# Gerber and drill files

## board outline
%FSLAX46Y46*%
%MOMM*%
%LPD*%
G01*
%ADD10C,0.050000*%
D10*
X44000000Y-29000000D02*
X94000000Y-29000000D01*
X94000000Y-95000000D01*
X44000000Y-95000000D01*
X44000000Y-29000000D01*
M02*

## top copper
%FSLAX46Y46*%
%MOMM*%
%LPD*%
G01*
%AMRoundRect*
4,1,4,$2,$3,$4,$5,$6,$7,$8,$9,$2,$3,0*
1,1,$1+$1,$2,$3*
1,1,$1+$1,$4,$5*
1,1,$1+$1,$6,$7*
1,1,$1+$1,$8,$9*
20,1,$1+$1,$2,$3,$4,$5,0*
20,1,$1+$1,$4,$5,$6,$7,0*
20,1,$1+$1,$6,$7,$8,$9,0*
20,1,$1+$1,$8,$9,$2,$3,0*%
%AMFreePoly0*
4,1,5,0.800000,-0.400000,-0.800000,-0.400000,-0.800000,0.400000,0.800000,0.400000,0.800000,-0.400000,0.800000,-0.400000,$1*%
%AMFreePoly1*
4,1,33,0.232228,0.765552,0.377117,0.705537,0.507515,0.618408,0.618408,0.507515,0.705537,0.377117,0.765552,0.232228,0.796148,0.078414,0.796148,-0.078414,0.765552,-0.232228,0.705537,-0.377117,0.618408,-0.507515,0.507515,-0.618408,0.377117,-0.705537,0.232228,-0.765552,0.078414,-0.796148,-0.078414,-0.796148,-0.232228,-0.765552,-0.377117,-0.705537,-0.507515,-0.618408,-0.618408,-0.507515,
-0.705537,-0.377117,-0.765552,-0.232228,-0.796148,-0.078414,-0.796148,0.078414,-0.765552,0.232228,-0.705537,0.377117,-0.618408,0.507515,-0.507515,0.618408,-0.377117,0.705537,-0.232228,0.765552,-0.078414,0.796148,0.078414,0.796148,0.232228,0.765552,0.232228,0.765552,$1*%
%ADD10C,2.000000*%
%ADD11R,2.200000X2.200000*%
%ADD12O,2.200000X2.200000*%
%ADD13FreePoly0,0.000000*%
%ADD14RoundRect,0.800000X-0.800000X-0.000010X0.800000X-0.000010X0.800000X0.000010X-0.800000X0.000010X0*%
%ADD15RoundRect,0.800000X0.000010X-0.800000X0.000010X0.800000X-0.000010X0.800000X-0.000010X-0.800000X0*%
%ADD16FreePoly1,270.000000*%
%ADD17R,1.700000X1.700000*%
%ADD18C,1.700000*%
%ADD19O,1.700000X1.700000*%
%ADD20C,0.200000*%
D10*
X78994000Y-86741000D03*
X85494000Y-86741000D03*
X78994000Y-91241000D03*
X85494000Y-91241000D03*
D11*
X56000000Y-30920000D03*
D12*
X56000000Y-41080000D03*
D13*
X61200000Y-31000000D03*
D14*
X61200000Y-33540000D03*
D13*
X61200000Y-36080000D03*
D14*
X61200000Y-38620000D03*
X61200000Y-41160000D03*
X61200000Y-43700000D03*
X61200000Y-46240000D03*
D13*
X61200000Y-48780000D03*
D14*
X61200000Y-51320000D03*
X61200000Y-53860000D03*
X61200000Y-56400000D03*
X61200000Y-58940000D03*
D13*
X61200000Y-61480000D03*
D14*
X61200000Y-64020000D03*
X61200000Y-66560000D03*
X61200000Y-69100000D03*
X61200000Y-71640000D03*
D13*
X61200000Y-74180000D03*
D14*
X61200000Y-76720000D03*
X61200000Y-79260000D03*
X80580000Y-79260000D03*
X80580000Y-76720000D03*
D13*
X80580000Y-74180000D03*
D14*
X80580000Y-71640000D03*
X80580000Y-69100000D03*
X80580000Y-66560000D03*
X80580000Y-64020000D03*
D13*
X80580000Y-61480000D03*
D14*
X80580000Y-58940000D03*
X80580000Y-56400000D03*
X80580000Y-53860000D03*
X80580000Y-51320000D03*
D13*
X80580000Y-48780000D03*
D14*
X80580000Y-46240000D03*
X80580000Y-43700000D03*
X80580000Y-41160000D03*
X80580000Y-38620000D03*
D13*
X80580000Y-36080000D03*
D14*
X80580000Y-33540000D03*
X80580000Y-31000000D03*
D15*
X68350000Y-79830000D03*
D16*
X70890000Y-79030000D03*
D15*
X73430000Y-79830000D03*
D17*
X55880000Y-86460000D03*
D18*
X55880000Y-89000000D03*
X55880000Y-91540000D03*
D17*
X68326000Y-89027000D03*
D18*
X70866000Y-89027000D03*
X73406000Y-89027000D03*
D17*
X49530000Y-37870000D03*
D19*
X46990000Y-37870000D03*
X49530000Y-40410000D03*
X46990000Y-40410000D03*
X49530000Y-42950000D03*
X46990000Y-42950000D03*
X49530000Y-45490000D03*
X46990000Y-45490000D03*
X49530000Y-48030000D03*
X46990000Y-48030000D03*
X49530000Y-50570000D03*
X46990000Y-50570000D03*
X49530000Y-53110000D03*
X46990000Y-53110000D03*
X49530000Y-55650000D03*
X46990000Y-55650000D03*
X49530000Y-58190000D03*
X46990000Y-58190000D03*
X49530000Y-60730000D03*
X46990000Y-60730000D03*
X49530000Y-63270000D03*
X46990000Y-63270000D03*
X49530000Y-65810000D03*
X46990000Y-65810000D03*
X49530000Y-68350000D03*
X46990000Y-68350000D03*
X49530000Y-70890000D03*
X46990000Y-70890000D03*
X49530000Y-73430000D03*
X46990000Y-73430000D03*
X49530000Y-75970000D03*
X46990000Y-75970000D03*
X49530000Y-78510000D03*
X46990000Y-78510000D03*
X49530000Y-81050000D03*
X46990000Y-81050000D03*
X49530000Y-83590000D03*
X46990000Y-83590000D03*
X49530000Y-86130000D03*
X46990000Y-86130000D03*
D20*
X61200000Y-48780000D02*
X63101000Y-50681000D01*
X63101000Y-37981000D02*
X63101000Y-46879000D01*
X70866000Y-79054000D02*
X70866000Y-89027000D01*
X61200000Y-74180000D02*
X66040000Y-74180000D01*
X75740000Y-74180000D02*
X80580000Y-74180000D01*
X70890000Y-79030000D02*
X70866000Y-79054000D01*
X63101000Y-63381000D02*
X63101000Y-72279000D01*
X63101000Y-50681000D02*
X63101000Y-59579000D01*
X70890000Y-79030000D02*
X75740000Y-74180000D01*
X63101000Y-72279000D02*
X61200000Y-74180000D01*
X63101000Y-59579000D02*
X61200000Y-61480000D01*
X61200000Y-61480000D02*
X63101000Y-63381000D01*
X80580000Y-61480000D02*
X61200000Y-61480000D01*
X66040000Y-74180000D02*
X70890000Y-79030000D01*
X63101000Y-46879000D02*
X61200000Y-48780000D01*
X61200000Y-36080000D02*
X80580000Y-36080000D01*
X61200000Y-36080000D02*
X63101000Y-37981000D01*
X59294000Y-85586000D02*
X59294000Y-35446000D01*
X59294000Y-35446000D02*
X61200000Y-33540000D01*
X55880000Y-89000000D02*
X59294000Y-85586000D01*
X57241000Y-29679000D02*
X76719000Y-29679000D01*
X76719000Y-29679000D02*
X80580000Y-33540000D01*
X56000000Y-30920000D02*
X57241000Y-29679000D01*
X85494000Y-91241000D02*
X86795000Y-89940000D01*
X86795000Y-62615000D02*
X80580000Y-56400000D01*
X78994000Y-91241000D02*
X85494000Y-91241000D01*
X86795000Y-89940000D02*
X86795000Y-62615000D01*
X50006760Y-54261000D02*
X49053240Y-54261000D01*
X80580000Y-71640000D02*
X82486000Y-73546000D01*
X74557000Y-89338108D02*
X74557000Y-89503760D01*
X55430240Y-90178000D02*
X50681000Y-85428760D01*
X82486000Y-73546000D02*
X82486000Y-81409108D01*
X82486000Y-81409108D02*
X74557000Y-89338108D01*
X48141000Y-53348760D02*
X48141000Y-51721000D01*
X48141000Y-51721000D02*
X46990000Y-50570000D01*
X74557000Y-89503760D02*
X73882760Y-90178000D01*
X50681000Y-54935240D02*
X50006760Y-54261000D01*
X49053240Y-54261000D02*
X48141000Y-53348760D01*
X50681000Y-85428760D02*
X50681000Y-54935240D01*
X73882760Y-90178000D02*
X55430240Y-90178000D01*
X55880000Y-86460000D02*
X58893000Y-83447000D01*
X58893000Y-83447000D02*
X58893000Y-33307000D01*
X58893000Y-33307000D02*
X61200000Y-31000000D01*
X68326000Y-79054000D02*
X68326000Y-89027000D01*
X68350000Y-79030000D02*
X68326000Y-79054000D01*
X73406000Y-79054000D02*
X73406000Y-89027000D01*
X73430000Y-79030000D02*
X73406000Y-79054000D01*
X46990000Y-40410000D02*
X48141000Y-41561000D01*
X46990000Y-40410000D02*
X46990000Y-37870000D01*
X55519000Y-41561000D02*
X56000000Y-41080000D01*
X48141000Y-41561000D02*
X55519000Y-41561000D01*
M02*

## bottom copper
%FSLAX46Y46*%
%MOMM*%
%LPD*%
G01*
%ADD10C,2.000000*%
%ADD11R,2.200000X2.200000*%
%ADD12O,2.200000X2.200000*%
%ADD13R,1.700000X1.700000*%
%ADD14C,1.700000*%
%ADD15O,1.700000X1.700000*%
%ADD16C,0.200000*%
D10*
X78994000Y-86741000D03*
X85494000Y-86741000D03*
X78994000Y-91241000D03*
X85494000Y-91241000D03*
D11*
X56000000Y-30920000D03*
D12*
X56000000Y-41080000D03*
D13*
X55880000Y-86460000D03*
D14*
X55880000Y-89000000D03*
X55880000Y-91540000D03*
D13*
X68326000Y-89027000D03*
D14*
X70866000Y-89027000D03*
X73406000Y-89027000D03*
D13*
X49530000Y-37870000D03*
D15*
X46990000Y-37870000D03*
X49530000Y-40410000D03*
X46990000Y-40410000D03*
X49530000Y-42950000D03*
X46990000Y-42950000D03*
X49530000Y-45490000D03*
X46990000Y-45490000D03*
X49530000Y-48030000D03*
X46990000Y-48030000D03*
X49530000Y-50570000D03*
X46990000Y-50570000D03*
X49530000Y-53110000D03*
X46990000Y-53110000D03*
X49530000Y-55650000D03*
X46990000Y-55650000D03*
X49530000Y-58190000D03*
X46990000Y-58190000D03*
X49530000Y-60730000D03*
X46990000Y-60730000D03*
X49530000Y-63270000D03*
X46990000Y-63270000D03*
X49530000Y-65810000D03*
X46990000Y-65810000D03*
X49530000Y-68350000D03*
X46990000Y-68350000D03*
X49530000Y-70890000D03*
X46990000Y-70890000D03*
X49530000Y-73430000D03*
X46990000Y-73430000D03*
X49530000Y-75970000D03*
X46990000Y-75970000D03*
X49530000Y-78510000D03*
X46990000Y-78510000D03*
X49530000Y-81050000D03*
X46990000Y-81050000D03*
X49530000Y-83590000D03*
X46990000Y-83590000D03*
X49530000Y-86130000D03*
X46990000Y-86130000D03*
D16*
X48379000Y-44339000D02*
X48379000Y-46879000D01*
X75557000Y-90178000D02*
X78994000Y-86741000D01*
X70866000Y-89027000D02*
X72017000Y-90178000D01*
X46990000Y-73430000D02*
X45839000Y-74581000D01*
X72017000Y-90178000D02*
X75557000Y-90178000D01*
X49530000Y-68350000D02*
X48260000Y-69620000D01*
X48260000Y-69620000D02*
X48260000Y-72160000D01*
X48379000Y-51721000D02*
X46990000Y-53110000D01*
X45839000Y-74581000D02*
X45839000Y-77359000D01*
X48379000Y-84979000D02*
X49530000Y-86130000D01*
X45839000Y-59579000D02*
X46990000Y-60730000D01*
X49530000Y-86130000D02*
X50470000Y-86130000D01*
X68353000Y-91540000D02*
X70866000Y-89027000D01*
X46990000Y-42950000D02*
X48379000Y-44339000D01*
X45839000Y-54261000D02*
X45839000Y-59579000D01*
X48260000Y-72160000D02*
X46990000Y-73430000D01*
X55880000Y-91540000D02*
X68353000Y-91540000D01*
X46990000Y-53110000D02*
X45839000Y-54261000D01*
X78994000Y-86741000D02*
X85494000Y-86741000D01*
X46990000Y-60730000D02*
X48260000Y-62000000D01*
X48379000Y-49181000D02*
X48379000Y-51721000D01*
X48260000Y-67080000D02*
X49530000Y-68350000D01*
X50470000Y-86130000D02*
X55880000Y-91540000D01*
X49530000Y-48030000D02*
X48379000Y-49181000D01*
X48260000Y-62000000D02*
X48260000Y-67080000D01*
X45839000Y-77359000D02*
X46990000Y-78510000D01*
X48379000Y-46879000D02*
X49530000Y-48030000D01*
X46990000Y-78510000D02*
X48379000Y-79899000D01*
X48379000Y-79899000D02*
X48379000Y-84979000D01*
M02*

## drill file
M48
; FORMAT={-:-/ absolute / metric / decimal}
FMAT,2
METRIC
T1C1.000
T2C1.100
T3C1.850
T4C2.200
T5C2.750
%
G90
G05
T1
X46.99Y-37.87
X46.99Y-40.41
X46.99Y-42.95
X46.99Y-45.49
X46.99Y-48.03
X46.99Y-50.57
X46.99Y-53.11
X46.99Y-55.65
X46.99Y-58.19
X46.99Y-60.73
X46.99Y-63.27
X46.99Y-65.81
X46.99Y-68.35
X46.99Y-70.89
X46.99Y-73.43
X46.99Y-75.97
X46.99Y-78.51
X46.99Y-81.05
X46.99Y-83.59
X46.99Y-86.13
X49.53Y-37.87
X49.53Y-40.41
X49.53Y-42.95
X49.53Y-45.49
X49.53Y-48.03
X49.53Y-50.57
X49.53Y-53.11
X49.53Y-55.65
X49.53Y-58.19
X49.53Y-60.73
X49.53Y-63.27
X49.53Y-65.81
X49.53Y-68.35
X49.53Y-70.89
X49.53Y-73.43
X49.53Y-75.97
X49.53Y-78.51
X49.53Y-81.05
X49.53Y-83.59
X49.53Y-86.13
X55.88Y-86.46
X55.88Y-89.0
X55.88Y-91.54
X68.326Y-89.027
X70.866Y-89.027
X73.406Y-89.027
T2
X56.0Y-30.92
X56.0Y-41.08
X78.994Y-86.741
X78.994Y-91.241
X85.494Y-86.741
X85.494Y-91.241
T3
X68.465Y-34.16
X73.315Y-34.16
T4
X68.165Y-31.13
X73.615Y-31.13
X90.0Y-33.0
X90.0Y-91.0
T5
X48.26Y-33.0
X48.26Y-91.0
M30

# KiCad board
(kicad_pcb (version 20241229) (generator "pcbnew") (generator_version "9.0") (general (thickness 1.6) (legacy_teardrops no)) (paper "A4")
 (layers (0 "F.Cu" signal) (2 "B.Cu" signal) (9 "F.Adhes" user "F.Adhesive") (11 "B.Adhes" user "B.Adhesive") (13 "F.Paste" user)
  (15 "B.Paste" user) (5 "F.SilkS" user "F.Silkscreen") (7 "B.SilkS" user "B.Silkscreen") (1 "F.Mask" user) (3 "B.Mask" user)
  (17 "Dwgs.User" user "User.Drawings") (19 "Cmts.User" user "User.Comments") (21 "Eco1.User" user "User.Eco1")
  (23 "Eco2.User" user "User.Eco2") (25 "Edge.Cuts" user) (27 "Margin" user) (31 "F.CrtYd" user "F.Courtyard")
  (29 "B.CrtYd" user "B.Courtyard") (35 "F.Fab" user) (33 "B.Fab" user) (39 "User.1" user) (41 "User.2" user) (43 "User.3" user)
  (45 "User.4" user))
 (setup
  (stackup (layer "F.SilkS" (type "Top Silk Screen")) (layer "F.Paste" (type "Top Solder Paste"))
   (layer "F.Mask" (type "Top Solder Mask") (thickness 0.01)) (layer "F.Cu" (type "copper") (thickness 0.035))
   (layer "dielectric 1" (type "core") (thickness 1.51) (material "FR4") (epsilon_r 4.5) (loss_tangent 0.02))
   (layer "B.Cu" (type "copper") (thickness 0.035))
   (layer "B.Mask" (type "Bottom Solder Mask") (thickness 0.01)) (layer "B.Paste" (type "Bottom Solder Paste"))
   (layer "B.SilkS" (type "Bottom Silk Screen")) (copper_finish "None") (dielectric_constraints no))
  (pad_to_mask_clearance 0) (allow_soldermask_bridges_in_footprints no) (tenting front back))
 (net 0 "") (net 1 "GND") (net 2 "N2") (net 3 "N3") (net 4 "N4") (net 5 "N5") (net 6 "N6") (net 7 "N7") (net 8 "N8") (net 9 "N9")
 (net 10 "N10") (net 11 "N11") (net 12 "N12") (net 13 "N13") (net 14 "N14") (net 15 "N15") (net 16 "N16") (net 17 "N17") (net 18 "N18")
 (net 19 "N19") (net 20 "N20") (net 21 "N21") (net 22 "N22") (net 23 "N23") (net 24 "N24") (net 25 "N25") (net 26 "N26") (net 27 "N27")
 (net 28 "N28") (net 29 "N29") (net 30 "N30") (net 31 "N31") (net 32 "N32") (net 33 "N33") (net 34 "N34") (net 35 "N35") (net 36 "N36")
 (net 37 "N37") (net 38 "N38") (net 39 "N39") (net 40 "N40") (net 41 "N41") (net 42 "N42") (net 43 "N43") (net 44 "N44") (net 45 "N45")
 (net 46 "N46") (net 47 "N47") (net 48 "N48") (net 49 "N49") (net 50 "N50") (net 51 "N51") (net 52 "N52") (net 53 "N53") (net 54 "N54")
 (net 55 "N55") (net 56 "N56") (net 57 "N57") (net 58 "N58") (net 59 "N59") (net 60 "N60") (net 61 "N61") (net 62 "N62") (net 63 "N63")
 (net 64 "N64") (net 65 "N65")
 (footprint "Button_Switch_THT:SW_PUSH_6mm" (layer "F.Cu") (at 78.994 86.741)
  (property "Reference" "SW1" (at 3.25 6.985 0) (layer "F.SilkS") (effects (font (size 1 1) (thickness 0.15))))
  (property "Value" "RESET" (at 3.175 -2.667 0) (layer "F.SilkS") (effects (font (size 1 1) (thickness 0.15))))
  (pad "1" thru_hole circle (at 0 0 90) (size 2 2) (drill 1.1) (layers "*.Cu" "*.Mask") (remove_unused_layers no) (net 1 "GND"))
  (pad "1" thru_hole circle (at 6.5 0 90) (size 2 2) (drill 1.1) (layers "*.Cu" "*.Mask") (remove_unused_layers no) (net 1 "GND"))
  (pad "2" thru_hole circle (at 0 4.5 90) (size 2 2) (drill 1.1) (layers "*.Cu" "*.Mask") (remove_unused_layers no) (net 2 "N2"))
  (pad "2" thru_hole circle (at 6.5 4.5 90) (size 2 2) (drill 1.1) (layers "*.Cu" "*.Mask") (remove_unused_layers no) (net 2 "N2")))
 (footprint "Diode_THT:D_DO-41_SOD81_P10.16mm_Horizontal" (layer "F.Cu") (at 56 30.92 -90)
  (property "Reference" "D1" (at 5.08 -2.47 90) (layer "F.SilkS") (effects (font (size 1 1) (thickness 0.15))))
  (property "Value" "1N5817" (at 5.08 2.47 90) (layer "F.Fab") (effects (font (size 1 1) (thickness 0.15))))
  (pad "1" thru_hole rect (at 0 0 270) (size 2.2 2.2) (drill 1.1) (layers "*.Cu" "*.Mask") (remove_unused_layers no) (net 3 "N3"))
  (pad "2" thru_hole oval (at 10.16 0 270) (size 2.2 2.2) (drill 1.1) (layers "*.Cu" "*.Mask") (remove_unused_layers no) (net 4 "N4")))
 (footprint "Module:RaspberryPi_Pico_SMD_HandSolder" (layer "F.Cu") (at 70.89 55.13)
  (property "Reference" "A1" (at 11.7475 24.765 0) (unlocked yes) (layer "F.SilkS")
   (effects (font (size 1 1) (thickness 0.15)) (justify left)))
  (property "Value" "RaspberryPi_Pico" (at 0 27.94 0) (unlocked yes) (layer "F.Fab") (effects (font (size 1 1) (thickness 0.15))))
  (pad "" smd rect (at -8.89 -24.13) (size 3.8 2.2) (drill (offset -0.8 0)) (layers "F.Paste"))
  (pad "" smd rect (at -8.89 -21.59) (size 3.8 2.2) (drill (offset -0.8 0)) (layers "F.Paste"))
  (pad "" smd rect (at -8.89 -19.05) (size 3.8 2.2) (drill (offset -0.8 0)) (layers "F.Paste"))
  (pad "" smd rect (at -8.89 -16.51) (size 3.8 2.2) (drill (offset -0.8 0)) (layers "F.Paste"))
  (pad "" smd rect (at -8.89 -13.97) (size 3.8 2.2) (drill (offset -0.8 0)) (layers "F.Paste"))
  (pad "" smd rect (at -8.89 -11.43) (size 3.8 2.2) (drill (offset -0.8 0)) (layers "F.Paste"))
  (pad "" smd rect (at -8.89 -8.89) (size 3.8 2.2) (drill (offset -0.8 0)) (layers "F.Paste"))
  (pad "" smd rect (at -8.89 -6.35) (size 3.8 2.2) (drill (offset -0.8 0)) (layers "F.Paste"))
  (pad "" smd rect (at -8.89 -3.81) (size 3.8 2.2) (drill (offset -0.8 0)) (layers "F.Paste"))
  (pad "" smd rect (at -8.89 -1.27) (size 3.8 2.2) (drill (offset -0.8 0)) (layers "F.Paste"))
  (pad "" smd rect (at -8.89 1.27) (size 3.8 2.2) (drill (offset -0.8 0)) (layers "F.Paste"))
  (pad "" smd rect (at -8.89 3.81) (size 3.8 2.2) (drill (offset -0.8 0)) (layers "F.Paste"))
  (pad "" smd rect (at -8.89 6.35) (size 3.8 2.2) (drill (offset -0.8 0)) (layers "F.Paste"))
  (pad "" smd rect (at -8.89 8.89) (size 3.8 2.2) (drill (offset -0.8 0)) (layers "F.Paste"))
  (pad "" smd rect (at -8.89 11.43) (size 3.8 2.2) (drill (offset -0.8 0)) (layers "F.Paste"))
  (pad "" smd rect (at -8.89 13.97) (size 3.8 2.2) (drill (offset -0.8 0)) (layers "F.Paste"))
  (pad "" smd rect (at -8.89 16.51) (size 3.8 2.2) (drill (offset -0.8 0)) (layers "F.Paste"))
  (pad "" smd rect (at -8.89 19.05) (size 3.8 2.2) (drill (offset -0.8 0)) (layers "F.Paste"))
  (pad "" smd rect (at -8.89 21.59) (size 3.8 2.2) (drill (offset -0.8 0)) (layers "F.Paste"))
  (pad "" smd rect (at -8.89 24.13) (size 3.8 2.2) (drill (offset -0.8 0)) (layers "F.Paste"))
  (pad "" np_thru_hole circle (at -2.725 -24) (size 2.2 2.2) (drill 2.2) (layers "*.Mask"))
  (pad "" smd rect (at -2.54 23.9) (size 2.2 3.8) (drill (offset 0 0.8)) (layers "F.Paste"))
  (pad "" np_thru_hole circle (at -2.425 -20.97) (size 1.85 1.85) (drill 1.85) (layers "*.Mask"))
  (pad "" smd rect (at 0 23.9) (size 2.2 3.8) (drill (offset 0 0.8)) (layers "F.Paste"))
  (pad "" np_thru_hole circle (at 2.425 -20.97) (size 1.85 1.85) (drill 1.85) (layers "*.Mask"))
  (pad "" smd rect (at 2.54 23.9) (size 2.2 3.8) (drill (offset 0 0.8)) (layers "F.Paste"))
  (pad "" np_thru_hole circle (at 2.725 -24) (size 2.2 2.2) (drill 2.2) (layers "*.Mask"))
  (pad "" smd rect (at 8.89 -24.13) (size 3.8 2.2) (drill (offset 0.8 0)) (layers "F.Paste"))
  (pad "" smd rect (at 8.89 -21.59) (size 3.8 2.2) (drill (offset 0.8 0)) (layers "F.Paste"))
  (pad "" smd rect (at 8.89 -19.05) (size 3.8 2.2) (drill (offset 0.8 0)) (layers "F.Paste"))
  (pad "" smd rect (at 8.89 -16.51) (size 3.8 2.2) (drill (offset 0.8 0)) (layers "F.Paste"))
  (pad "" smd rect (at 8.89 -13.97) (size 3.8 2.2) (drill (offset 0.8 0)) (layers "F.Paste"))
  (pad "" smd rect (at 8.89 -11.43) (size 3.8 2.2) (drill (offset 0.8 0)) (layers "F.Paste"))
  (pad "" smd rect (at 8.89 -8.89) (size 3.8 2.2) (drill (offset 0.8 0)) (layers "F.Paste"))
  (pad "" smd rect (at 8.89 -6.35) (size 3.8 2.2) (drill (offset 0.8 0)) (layers "F.Paste"))
  (pad "" smd rect (at 8.89 -3.81) (size 3.8 2.2) (drill (offset 0.8 0)) (layers "F.Paste"))
  (pad "" smd rect (at 8.89 -1.27) (size 3.8 2.2) (drill (offset 0.8 0)) (layers "F.Paste"))
  (pad "" smd rect (at 8.89 1.27) (size 3.8 2.2) (drill (offset 0.8 0)) (layers "F.Paste"))
  (pad "" smd rect (at 8.89 3.81) (size 3.8 2.2) (drill (offset 0.8 0)) (layers "F.Paste"))
  (pad "" smd rect (at 8.89 6.35) (size 3.8 2.2) (drill (offset 0.8 0)) (layers "F.Paste"))
  (pad "" smd rect (at 8.89 8.89) (size 3.8 2.2) (drill (offset 0.8 0)) (layers "F.Paste"))
  (pad "" smd rect (at 8.89 11.43) (size 3.8 2.2) (drill (offset 0.8 0)) (layers "F.Paste"))
  (pad "" smd rect (at 8.89 13.97) (size 3.8 2.2) (drill (offset 0.8 0)) (layers "F.Paste"))
  (pad "" smd rect (at 8.89 16.51) (size 3.8 2.2) (drill (offset 0.8 0)) (layers "F.Paste"))
  (pad "" smd rect (at 8.89 19.05) (size 3.8 2.2) (drill (offset 0.8 0)) (layers "F.Paste"))
  (pad "" smd rect (at 8.89 21.59) (size 3.8 2.2) (drill (offset 0.8 0)) (layers "F.Paste"))
  (pad "" smd rect (at 8.89 24.13) (size 3.8 2.2) (drill (offset 0.8 0)) (layers "F.Paste"))
  (pad "1" smd custom (at -9.69 -24.13) (size 1.6 0.8) (layers "F.Cu" "F.Mask") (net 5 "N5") (options (clearance outline) (anchor rect))
   (primitives))
  (pad "2" smd roundrect (at -9.69 -21.59) (size 3.2 1.6) (layers "F.Cu" "F.Mask") (roundrect_rratio 0.5) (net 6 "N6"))
  (pad "3" smd custom (at -9.69 -19.05) (size 1.6 0.8) (layers "F.Cu" "F.Mask") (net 1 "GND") (options (clearance outline) (anchor rect))
   (primitives))
  (pad "4" smd roundrect (at -9.69 -16.51) (size 3.2 1.6) (layers "F.Cu" "F.Mask") (roundrect_rratio 0.5) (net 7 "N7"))
  (pad "5" smd roundrect (at -9.69 -13.97) (size 3.2 1.6) (layers "F.Cu" "F.Mask") (roundrect_rratio 0.5) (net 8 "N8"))
  (pad "6" smd roundrect (at -9.69 -11.43) (size 3.2 1.6) (layers "F.Cu" "F.Mask") (roundrect_rratio 0.5) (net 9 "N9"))
  (pad "7" smd roundrect (at -9.69 -8.89) (size 3.2 1.6) (layers "F.Cu" "F.Mask") (roundrect_rratio 0.5) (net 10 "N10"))
  (pad "8" smd custom (at -9.69 -6.35) (size 1.6 0.8) (layers "F.Cu" "F.Mask") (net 1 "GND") (options (clearance outline) (anchor rect))
   (primitives))
  (pad "9" smd roundrect (at -9.69 -3.81) (size 3.2 1.6) (layers "F.Cu" "F.Mask") (roundrect_rratio 0.5) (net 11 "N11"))
  (pad "10" smd roundrect (at -9.69 -1.27) (size 3.2 1.6) (layers "F.Cu" "F.Mask") (roundrect_rratio 0.5) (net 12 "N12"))
  (pad "11" smd roundrect (at -9.69 1.27) (size 3.2 1.6) (layers "F.Cu" "F.Mask") (roundrect_rratio 0.5) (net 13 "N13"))
  (pad "12" smd roundrect (at -9.69 3.81) (size 3.2 1.6) (layers "F.Cu" "F.Mask") (roundrect_rratio 0.5) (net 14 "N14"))
  (pad "13" smd custom (at -9.69 6.35) (size 1.6 0.8) (layers "F.Cu" "F.Mask") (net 1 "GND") (options (clearance outline) (anchor rect))
   (primitives))
  (pad "14" smd roundrect (at -9.69 8.89) (size 3.2 1.6) (layers "F.Cu" "F.Mask") (roundrect_rratio 0.5) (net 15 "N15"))
  (pad "15" smd roundrect (at -9.69 11.43) (size 3.2 1.6) (layers "F.Cu" "F.Mask") (roundrect_rratio 0.5) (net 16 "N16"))
  (pad "16" smd roundrect (at -9.69 13.97) (size 3.2 1.6) (layers "F.Cu" "F.Mask") (roundrect_rratio 0.5) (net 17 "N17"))
  (pad "17" smd roundrect (at -9.69 16.51) (size 3.2 1.6) (layers "F.Cu" "F.Mask") (roundrect_rratio 0.5) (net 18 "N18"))
  (pad "18" smd custom (at -9.69 19.05) (size 1.6 0.8) (layers "F.Cu" "F.Mask") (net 1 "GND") (options (clearance outline) (anchor rect))
   (primitives))
  (pad "19" smd roundrect (at -9.69 21.59) (size 3.2 1.6) (layers "F.Cu" "F.Mask") (roundrect_rratio 0.5) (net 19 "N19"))
  (pad "20" smd roundrect (at -9.69 24.13) (size 3.2 1.6) (layers "F.Cu" "F.Mask") (roundrect_rratio 0.5) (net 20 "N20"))
  (pad "21" smd roundrect (at 9.69 24.13) (size 3.2 1.6) (layers "F.Cu" "F.Mask") (roundrect_rratio 0.5) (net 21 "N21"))
  (pad "22" smd roundrect (at 9.69 21.59) (size 3.2 1.6) (layers "F.Cu" "F.Mask") (roundrect_rratio 0.5) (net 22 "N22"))
  (pad "23" smd custom (at 9.69 19.05) (size 1.6 0.8) (layers "F.Cu" "F.Mask") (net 1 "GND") (options (clearance outline) (anchor rect))
   (primitives))
  (pad "24" smd roundrect (at 9.69 16.51) (size 3.2 1.6) (layers "F.Cu" "F.Mask") (roundrect_rratio 0.5) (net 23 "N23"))
  (pad "25" smd roundrect (at 9.69 13.97) (size 3.2 1.6) (layers "F.Cu" "F.Mask") (roundrect_rratio 0.5) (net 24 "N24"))
  (pad "26" smd roundrect (at 9.69 11.43) (size 3.2 1.6) (layers "F.Cu" "F.Mask") (roundrect_rratio 0.5) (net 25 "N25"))
  (pad "27" smd roundrect (at 9.69 8.89) (size 3.2 1.6) (layers "F.Cu" "F.Mask") (roundrect_rratio 0.5) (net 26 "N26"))
  (pad "28" smd custom (at 9.69 6.35) (size 1.6 0.8) (layers "F.Cu" "F.Mask") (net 1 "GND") (options (clearance outline) (anchor rect))
   (primitives))
  (pad "29" smd roundrect (at 9.69 3.81) (size 3.2 1.6) (layers "F.Cu" "F.Mask") (roundrect_rratio 0.5) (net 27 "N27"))
  (pad "30" smd roundrect (at 9.69 1.27) (size 3.2 1.6) (layers "F.Cu" "F.Mask") (roundrect_rratio 0.5) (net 2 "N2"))
  (pad "31" smd roundrect (at 9.69 -1.27) (size 3.2 1.6) (layers "F.Cu" "F.Mask") (roundrect_rratio 0.5) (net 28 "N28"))
  (pad "32" smd roundrect (at 9.69 -3.81) (size 3.2 1.6) (layers "F.Cu" "F.Mask") (roundrect_rratio 0.5) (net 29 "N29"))
  (pad "33" smd custom (at 9.69 -6.35) (size 1.6 0.8) (layers "F.Cu" "F.Mask") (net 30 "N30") (options (clearance outline) (anchor rect))
   (primitives))
  (pad "34" smd roundrect (at 9.69 -8.89) (size 3.2 1.6) (layers "F.Cu" "F.Mask") (roundrect_rratio 0.5) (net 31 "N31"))
  (pad "35" smd roundrect (at 9.69 -11.43) (size 3.2 1.6) (layers "F.Cu" "F.Mask") (roundrect_rratio 0.5) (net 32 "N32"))
  (pad "36" smd roundrect (at 9.69 -13.97) (size 3.2 1.6) (layers "F.Cu" "F.Mask") (roundrect_rratio 0.5) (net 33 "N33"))
  (pad "37" smd roundrect (at 9.69 -16.51) (size 3.2 1.6) (layers "F.Cu" "F.Mask") (roundrect_rratio 0.5) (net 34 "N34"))
  (pad "38" smd custom (at 9.69 -19.05) (size 1.6 0.8) (layers "F.Cu" "F.Mask") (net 1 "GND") (options (clearance outline) (anchor rect))
   (primitives))
  (pad "39" smd roundrect (at 9.69 -21.59) (size 3.2 1.6) (layers "F.Cu" "F.Mask") (roundrect_rratio 0.5) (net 3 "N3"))
  (pad "40" smd roundrect (at 9.69 -24.13) (size 3.2 1.6) (layers "F.Cu" "F.Mask") (roundrect_rratio 0.5) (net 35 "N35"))
  (pad "D1" smd roundrect (at -2.54 23.9 90) (size 3.2 1.6) (drill (offset -0.8 0)) (layers "F.Cu" "F.Mask") (roundrect_rratio 0.5)
   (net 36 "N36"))
  (pad "D2" smd custom (at 0 23.9 270) (size 1.6 1.6) (layers "F.Cu" "F.Mask") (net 1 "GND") (options (clearance outline) (anchor circle))
   (primitives))
  (pad "D3" smd roundrect (at 2.54 23.9 90) (size 3.2 1.6) (drill (offset -0.8 0)) (layers "F.Cu" "F.Mask") (roundrect_rratio 0.5)
   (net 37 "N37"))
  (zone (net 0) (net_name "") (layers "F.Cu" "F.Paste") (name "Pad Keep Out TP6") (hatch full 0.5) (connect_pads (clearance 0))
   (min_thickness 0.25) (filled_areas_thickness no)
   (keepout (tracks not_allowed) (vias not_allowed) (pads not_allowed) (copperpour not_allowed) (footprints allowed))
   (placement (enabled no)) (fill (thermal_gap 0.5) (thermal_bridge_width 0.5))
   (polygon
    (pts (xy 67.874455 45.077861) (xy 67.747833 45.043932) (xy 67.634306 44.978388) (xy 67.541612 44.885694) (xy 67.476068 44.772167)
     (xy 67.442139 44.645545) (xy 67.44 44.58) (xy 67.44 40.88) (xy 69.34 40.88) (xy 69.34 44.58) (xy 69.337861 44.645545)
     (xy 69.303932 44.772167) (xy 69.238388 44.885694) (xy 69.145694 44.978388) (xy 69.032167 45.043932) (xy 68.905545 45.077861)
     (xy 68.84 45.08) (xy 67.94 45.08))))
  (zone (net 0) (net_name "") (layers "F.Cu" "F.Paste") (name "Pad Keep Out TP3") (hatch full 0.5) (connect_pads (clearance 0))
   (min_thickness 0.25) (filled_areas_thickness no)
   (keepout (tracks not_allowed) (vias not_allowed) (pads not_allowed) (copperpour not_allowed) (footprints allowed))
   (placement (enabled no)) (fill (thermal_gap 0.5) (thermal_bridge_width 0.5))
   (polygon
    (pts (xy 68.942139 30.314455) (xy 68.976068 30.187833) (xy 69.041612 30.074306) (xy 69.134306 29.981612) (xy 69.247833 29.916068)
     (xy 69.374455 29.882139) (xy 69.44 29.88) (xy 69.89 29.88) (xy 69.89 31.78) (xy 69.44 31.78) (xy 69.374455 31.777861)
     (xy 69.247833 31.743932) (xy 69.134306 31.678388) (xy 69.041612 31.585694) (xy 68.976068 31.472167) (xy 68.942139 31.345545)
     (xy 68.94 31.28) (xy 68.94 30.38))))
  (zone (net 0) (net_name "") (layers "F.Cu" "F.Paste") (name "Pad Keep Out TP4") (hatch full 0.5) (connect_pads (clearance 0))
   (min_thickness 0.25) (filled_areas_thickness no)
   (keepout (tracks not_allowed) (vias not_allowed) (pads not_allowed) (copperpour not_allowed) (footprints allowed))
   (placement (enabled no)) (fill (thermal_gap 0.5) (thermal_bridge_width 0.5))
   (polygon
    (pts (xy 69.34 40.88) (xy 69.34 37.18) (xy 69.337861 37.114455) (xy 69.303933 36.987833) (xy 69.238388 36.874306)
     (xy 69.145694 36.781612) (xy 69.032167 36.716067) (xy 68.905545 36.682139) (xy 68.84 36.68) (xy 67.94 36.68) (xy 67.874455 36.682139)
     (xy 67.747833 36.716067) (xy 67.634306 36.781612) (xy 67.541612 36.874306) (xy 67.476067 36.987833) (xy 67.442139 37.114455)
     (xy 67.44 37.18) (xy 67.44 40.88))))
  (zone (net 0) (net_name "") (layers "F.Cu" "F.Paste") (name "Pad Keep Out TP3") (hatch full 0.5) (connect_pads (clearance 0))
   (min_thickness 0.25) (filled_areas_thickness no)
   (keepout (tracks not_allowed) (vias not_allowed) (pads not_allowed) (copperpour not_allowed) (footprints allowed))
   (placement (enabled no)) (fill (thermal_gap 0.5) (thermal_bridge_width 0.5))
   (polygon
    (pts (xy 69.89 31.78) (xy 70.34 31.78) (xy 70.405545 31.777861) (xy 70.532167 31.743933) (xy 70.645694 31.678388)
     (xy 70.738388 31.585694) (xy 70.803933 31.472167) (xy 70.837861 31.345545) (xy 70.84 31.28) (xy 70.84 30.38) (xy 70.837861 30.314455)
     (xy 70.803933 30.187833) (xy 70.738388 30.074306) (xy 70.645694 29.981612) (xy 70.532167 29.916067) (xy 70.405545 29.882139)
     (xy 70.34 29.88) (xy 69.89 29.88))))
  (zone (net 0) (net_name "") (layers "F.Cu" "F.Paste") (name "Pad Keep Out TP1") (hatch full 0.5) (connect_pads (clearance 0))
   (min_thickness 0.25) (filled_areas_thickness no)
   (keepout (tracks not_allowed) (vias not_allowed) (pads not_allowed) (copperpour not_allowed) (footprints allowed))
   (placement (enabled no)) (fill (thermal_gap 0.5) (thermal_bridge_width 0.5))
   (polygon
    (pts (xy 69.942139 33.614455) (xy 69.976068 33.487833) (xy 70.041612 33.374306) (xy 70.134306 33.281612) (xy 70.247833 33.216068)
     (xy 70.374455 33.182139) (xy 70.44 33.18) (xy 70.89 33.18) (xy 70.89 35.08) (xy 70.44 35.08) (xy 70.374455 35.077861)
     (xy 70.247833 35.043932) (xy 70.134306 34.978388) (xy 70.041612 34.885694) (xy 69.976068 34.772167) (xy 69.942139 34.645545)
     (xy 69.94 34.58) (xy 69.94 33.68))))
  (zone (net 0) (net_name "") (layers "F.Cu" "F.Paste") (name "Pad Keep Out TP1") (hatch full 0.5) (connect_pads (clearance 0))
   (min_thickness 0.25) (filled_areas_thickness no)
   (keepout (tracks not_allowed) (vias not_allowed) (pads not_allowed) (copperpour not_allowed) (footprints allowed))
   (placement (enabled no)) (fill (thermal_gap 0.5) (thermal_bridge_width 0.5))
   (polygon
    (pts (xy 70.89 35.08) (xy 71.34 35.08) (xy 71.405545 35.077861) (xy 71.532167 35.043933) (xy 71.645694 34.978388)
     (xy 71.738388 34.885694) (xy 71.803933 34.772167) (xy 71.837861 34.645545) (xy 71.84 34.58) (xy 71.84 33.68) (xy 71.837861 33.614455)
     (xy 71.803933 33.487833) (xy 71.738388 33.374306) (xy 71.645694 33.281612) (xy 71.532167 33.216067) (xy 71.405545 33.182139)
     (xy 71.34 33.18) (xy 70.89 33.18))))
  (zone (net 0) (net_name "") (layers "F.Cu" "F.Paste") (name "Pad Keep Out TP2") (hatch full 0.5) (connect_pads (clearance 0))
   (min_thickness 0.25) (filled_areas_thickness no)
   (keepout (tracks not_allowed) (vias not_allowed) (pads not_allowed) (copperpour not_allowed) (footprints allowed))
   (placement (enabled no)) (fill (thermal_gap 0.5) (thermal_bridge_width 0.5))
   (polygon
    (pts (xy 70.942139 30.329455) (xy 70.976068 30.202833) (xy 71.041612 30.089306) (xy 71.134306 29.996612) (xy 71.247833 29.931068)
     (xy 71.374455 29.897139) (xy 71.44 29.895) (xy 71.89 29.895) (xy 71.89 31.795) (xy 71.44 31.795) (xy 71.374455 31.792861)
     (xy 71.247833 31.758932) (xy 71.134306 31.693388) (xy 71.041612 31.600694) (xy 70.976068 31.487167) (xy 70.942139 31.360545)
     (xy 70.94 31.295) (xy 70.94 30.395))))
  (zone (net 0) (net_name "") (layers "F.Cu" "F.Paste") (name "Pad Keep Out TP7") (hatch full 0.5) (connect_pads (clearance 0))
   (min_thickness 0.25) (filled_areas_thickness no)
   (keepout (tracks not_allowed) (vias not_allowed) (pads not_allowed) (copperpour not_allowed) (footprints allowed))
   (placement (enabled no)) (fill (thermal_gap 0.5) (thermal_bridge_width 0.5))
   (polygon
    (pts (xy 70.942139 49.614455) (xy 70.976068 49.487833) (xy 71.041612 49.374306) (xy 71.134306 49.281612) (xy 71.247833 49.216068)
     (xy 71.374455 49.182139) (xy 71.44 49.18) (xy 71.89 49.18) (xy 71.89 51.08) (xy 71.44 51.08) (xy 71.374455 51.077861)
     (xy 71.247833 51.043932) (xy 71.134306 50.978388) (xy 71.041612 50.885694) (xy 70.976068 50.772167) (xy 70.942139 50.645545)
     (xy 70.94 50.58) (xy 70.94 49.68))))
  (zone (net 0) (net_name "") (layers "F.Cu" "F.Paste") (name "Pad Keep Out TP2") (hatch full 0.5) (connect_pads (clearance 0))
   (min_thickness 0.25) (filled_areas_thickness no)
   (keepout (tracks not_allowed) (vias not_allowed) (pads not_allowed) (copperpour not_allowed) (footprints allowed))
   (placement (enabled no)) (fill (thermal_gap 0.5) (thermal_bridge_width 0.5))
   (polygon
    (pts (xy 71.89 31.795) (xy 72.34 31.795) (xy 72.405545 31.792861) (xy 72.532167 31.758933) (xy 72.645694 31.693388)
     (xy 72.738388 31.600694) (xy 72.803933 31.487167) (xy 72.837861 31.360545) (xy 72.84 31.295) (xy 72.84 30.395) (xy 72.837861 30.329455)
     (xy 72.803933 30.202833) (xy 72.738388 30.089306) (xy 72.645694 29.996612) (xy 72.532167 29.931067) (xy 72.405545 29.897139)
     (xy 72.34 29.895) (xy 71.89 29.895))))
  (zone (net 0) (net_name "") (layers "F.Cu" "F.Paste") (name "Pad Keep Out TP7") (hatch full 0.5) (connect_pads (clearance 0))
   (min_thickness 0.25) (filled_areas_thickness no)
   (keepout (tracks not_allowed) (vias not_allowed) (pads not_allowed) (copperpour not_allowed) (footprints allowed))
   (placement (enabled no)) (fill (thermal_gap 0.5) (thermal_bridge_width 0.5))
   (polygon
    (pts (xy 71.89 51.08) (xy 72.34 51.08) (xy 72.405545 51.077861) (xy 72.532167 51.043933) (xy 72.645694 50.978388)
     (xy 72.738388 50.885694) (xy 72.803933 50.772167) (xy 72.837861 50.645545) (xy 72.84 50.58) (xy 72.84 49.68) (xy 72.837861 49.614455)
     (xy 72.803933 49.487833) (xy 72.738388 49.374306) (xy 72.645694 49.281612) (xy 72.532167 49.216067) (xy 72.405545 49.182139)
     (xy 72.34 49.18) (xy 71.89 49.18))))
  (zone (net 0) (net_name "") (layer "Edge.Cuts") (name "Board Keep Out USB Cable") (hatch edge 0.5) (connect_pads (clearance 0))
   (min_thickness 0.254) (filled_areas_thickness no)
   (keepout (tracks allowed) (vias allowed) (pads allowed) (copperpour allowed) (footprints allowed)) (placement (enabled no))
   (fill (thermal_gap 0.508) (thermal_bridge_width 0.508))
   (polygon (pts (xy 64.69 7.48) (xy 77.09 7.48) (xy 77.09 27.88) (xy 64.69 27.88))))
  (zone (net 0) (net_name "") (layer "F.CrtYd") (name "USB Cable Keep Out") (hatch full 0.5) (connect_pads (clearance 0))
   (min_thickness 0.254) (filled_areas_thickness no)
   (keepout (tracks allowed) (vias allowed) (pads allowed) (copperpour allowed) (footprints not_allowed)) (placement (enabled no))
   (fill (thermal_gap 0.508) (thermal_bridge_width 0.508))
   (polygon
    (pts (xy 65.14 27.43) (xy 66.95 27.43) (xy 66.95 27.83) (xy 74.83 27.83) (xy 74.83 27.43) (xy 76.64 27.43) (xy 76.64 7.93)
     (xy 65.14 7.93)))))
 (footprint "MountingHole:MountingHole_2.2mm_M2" (layer "F.Cu") (at 90 91)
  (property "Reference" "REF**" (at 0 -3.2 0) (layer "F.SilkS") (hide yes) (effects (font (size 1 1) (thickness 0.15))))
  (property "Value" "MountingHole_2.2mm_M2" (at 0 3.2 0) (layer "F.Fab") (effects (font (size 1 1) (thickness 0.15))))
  (pad "" np_thru_hole circle (at 0 0) (size 2.2 2.2) (drill 2.2) (layers "*.Cu" "*.Mask")))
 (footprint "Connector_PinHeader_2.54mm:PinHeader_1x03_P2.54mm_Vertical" (layer "F.Cu") (at 55.88 86.46)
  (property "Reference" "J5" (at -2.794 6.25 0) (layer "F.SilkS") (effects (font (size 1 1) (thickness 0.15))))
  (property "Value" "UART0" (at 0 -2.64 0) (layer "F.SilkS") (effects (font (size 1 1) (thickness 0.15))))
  (pad "1" thru_hole rect (at 0 0) (size 1.7 1.7) (drill 1) (layers "*.Cu" "*.Mask") (remove_unused_layers no) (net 5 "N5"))
  (pad "2" thru_hole circle (at 0 2.54) (size 1.7 1.7) (drill 1) (layers "*.Cu" "*.Mask") (remove_unused_layers no) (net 6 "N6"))
  (pad "3" thru_hole circle (at 0 5.08) (size 1.7 1.7) (drill 1) (layers "*.Cu" "*.Mask") (remove_unused_layers no) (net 1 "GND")))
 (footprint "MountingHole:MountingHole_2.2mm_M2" (layer "F.Cu") (at 90 33)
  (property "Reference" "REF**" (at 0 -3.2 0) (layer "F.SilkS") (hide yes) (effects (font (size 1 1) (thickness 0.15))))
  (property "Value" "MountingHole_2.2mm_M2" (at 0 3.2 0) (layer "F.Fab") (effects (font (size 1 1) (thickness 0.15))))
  (pad "" np_thru_hole circle (at 0 0) (size 2.2 2.2) (drill 2.2) (layers "*.Cu" "*.Mask")))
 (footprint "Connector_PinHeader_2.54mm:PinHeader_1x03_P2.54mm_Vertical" (layer "F.Cu") (at 68.326 89.027 90)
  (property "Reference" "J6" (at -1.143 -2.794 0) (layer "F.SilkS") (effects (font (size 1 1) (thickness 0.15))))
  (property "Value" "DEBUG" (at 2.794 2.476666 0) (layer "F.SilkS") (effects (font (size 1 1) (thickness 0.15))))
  (pad "1" thru_hole rect (at 0 0 90) (size 1.7 1.7) (drill 1) (layers "*.Cu" "*.Mask") (remove_unused_layers no) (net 36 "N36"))
  (pad "2" thru_hole circle (at 0 2.54 90) (size 1.7 1.7) (drill 1) (layers "*.Cu" "*.Mask") (remove_unused_layers no) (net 1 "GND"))
  (pad "3" thru_hole circle (at 0 5.08 90) (size 1.7 1.7) (drill 1) (layers "*.Cu" "*.Mask") (remove_unused_layers no) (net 37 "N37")))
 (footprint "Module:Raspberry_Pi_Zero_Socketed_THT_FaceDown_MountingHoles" (layer "F.Cu") (at 49.53 37.87)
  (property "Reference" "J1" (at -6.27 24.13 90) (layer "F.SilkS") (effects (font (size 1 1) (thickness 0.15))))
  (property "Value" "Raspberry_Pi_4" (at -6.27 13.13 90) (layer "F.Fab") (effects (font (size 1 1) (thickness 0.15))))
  (pad "" np_thru_hole circle (at -1.27 -4.87 90) (size 2.75 2.75) (drill 2.75) (layers "*.Cu" "*.Mask") (solder_mask_margin 1.625))
  (pad "" np_thru_hole circle (at -1.27 53.13 90) (size 2.75 2.75) (drill 2.75) (layers "*.Cu" "*.Mask") (solder_mask_margin 1.625))
  (pad "1" thru_hole rect (at 0 0) (size 1.7 1.7) (drill 1) (layers "*.Cu" "*.Mask") (remove_unused_layers no) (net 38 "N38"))
  (pad "2" thru_hole oval (at -2.54 0) (size 1.7 1.7) (drill 1) (layers "*.Cu" "*.Mask") (remove_unused_layers no) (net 4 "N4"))
  (pad "3" thru_hole oval (at 0 2.54) (size 1.7 1.7) (drill 1) (layers "*.Cu" "*.Mask") (remove_unused_layers no) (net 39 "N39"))
  (pad "4" thru_hole oval (at -2.54 2.54) (size 1.7 1.7) (drill 1) (layers "*.Cu" "*.Mask") (remove_unused_layers no) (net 4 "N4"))
  (pad "5" thru_hole oval (at 0 5.08) (size 1.7 1.7) (drill 1) (layers "*.Cu" "*.Mask") (remove_unused_layers no) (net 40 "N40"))
  (pad "6" thru_hole oval (at -2.54 5.08) (size 1.7 1.7) (drill 1) (layers "*.Cu" "*.Mask") (remove_unused_layers no) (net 1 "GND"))
  (pad "7" thru_hole oval (at 0 7.62) (size 1.7 1.7) (drill 1) (layers "*.Cu" "*.Mask") (remove_unused_layers no) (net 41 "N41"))
  (pad "8" thru_hole oval (at -2.54 7.62) (size 1.7 1.7) (drill 1) (layers "*.Cu" "*.Mask") (remove_unused_layers no) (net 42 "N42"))
  (pad "9" thru_hole oval (at 0 10.16) (size 1.7 1.7) (drill 1) (layers "*.Cu" "*.Mask") (remove_unused_layers no) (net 1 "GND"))
  (pad "10" thru_hole oval (at -2.54 10.16) (size 1.7 1.7) (drill 1) (layers "*.Cu" "*.Mask") (remove_unused_layers no) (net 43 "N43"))
  (pad "11" thru_hole oval (at 0 12.7) (size 1.7 1.7) (drill 1) (layers "*.Cu" "*.Mask") (remove_unused_layers no) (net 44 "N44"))
  (pad "12" thru_hole oval (at -2.54 12.7) (size 1.7 1.7) (drill 1) (layers "*.Cu" "*.Mask") (remove_unused_layers no) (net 23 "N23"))
  (pad "13" thru_hole oval (at 0 15.24) (size 1.7 1.7) (drill 1) (layers "*.Cu" "*.Mask") (remove_unused_layers no) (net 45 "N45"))
  (pad "14" thru_hole oval (at -2.54 15.24) (size 1.7 1.7) (drill 1) (layers "*.Cu" "*.Mask") (remove_unused_layers no) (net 1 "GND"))
  (pad "15" thru_hole oval (at 0 17.78) (size 1.7 1.7) (drill 1) (layers "*.Cu" "*.Mask") (remove_unused_layers no) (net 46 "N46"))
  (pad "16" thru_hole oval (at -2.54 17.78) (size 1.7 1.7) (drill 1) (layers "*.Cu" "*.Mask") (remove_unused_layers no) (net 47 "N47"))
  (pad "17" thru_hole oval (at 0 20.32) (size 1.7 1.7) (drill 1) (layers "*.Cu" "*.Mask") (remove_unused_layers no) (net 38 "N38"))
  (pad "18" thru_hole oval (at -2.54 20.32) (size 1.7 1.7) (drill 1) (layers "*.Cu" "*.Mask") (remove_unused_layers no) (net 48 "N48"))
  (pad "19" thru_hole oval (at 0 22.86) (size 1.7 1.7) (drill 1) (layers "*.Cu" "*.Mask") (remove_unused_layers no) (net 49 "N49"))
  (pad "20" thru_hole oval (at -2.54 22.86) (size 1.7 1.7) (drill 1) (layers "*.Cu" "*.Mask") (remove_unused_layers no) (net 1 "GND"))
  (pad "21" thru_hole oval (at 0 25.4) (size 1.7 1.7) (drill 1) (layers "*.Cu" "*.Mask") (remove_unused_layers no) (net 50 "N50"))
  (pad "22" thru_hole oval (at -2.54 25.4) (size 1.7 1.7) (drill 1) (layers "*.Cu" "*.Mask") (remove_unused_layers no) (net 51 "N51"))
  (pad "23" thru_hole oval (at 0 27.94) (size 1.7 1.7) (drill 1) (layers "*.Cu" "*.Mask") (remove_unused_layers no) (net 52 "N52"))
  (pad "24" thru_hole oval (at -2.54 27.94) (size 1.7 1.7) (drill 1) (layers "*.Cu" "*.Mask") (remove_unused_layers no) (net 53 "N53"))
  (pad "25" thru_hole oval (at 0 30.48) (size 1.7 1.7) (drill 1) (layers "*.Cu" "*.Mask") (remove_unused_layers no) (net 1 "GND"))
  (pad "26" thru_hole oval (at -2.54 30.48) (size 1.7 1.7) (drill 1) (layers "*.Cu" "*.Mask") (remove_unused_layers no) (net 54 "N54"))
  (pad "27" thru_hole oval (at 0 33.02) (size 1.7 1.7) (drill 1) (layers "*.Cu" "*.Mask") (remove_unused_layers no) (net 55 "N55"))
  (pad "28" thru_hole oval (at -2.54 33.02) (size 1.7 1.7) (drill 1) (layers "*.Cu" "*.Mask") (remove_unused_layers no) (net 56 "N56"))
  (pad "29" thru_hole oval (at 0 35.56) (size 1.7 1.7) (drill 1) (layers "*.Cu" "*.Mask") (remove_unused_layers no) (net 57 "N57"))
  (pad "30" thru_hole oval (at -2.54 35.56) (size 1.7 1.7) (drill 1) (layers "*.Cu" "*.Mask") (remove_unused_layers no) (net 1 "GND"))
  (pad "31" thru_hole oval (at 0 38.1) (size 1.7 1.7) (drill 1) (layers "*.Cu" "*.Mask") (remove_unused_layers no) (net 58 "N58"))
  (pad "32" thru_hole oval (at -2.54 38.1) (size 1.7 1.7) (drill 1) (layers "*.Cu" "*.Mask") (remove_unused_layers no) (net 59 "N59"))
  (pad "33" thru_hole oval (at 0 40.64) (size 1.7 1.7) (drill 1) (layers "*.Cu" "*.Mask") (remove_unused_layers no) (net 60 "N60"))
  (pad "34" thru_hole oval (at -2.54 40.64) (size 1.7 1.7) (drill 1) (layers "*.Cu" "*.Mask") (remove_unused_layers no) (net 1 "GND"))
  (pad "35" thru_hole oval (at 0 43.18) (size 1.7 1.7) (drill 1) (layers "*.Cu" "*.Mask") (remove_unused_layers no) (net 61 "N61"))
  (pad "36" thru_hole oval (at -2.54 43.18) (size 1.7 1.7) (drill 1) (layers "*.Cu" "*.Mask") (remove_unused_layers no) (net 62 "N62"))
  (pad "37" thru_hole oval (at 0 45.72) (size 1.7 1.7) (drill 1) (layers "*.Cu" "*.Mask") (remove_unused_layers no) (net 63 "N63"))
  (pad "38" thru_hole oval (at -2.54 45.72) (size 1.7 1.7) (drill 1) (layers "*.Cu" "*.Mask") (remove_unused_layers no) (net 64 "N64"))
  (pad "39" thru_hole oval (at 0 48.26) (size 1.7 1.7) (drill 1) (layers "*.Cu" "*.Mask") (remove_unused_layers no) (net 1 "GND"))
  (pad "40" thru_hole oval (at -2.54 48.26) (size 1.7 1.7) (drill 1) (layers "*.Cu" "*.Mask") (remove_unused_layers no) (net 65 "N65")))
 (gr_rect (start 44 29) (end 94 95) (stroke (width 0.05) (type default)) (fill no) (layer "Edge.Cuts"))
 (segment (start 61.2 48.78) (end 63.101 50.681) (width 0.2) (layer "F.Cu") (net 1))
 (segment (start 63.101 37.981) (end 63.101 46.879) (width 0.2) (layer "F.Cu") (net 1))
 (segment (start 70.866 79.054) (end 70.866 89.027) (width 0.2) (layer "F.Cu") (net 1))
 (segment (start 61.2 74.18) (end 66.04 74.18) (width 0.2) (layer "F.Cu") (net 1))
 (segment (start 75.74 74.18) (end 80.58 74.18) (width 0.2) (layer "F.Cu") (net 1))
 (segment (start 70.89 79.03) (end 70.866 79.054) (width 0.2) (layer "F.Cu") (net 1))
 (segment (start 63.101 63.381) (end 63.101 72.279) (width 0.2) (layer "F.Cu") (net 1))
 (segment (start 63.101 50.681) (end 63.101 59.579) (width 0.2) (layer "F.Cu") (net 1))
 (segment (start 70.89 79.03) (end 75.74 74.18) (width 0.2) (layer "F.Cu") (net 1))
 (segment (start 63.101 72.279) (end 61.2 74.18) (width 0.2) (layer "F.Cu") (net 1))
 (segment (start 63.101 59.579) (end 61.2 61.48) (width 0.2) (layer "F.Cu") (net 1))
 (segment (start 61.2 61.48) (end 63.101 63.381) (width 0.2) (layer "F.Cu") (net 1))
 (segment (start 80.58 61.48) (end 61.2 61.48) (width 0.2) (layer "F.Cu") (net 1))
 (segment (start 66.04 74.18) (end 70.89 79.03) (width 0.2) (layer "F.Cu") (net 1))
 (segment (start 63.101 46.879) (end 61.2 48.78) (width 0.2) (layer "F.Cu") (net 1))
 (segment (start 61.2 36.08) (end 80.58 36.08) (width 0.2) (layer "F.Cu") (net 1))
 (segment (start 61.2 36.08) (end 63.101 37.981) (width 0.2) (layer "F.Cu") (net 1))
 (segment (start 48.379 44.339) (end 48.379 46.879) (width 0.2) (layer "B.Cu") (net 1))
 (segment (start 75.557 90.178) (end 78.994 86.741) (width 0.2) (layer "B.Cu") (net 1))
 (segment (start 70.866 89.027) (end 72.017 90.178) (width 0.2) (layer "B.Cu") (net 1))
 (segment (start 46.99 73.43) (end 45.839 74.581) (width 0.2) (layer "B.Cu") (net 1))
 (segment (start 72.017 90.178) (end 75.557 90.178) (width 0.2) (layer "B.Cu") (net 1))
 (segment (start 49.53 68.35) (end 48.26 69.62) (width 0.2) (layer "B.Cu") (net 1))
 (segment (start 48.26 69.62) (end 48.26 72.16) (width 0.2) (layer "B.Cu") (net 1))
 (segment (start 48.379 51.721) (end 46.99 53.11) (width 0.2) (layer "B.Cu") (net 1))
 (segment (start 45.839 74.581) (end 45.839 77.359) (width 0.2) (layer "B.Cu") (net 1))
 (segment (start 48.379 84.979) (end 49.53 86.13) (width 0.2) (layer "B.Cu") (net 1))
 (segment (start 45.839 59.579) (end 46.99 60.73) (width 0.2) (layer "B.Cu") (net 1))
 (segment (start 49.53 86.13) (end 50.47 86.13) (width 0.2) (layer "B.Cu") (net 1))
 (segment (start 68.353 91.54) (end 70.866 89.027) (width 0.2) (layer "B.Cu") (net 1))
 (segment (start 46.99 42.95) (end 48.379 44.339) (width 0.2) (layer "B.Cu") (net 1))
 (segment (start 45.839 54.261) (end 45.839 59.579) (width 0.2) (layer "B.Cu") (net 1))
 (segment (start 48.26 72.16) (end 46.99 73.43) (width 0.2) (layer "B.Cu") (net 1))
 (segment (start 55.88 91.54) (end 68.353 91.54) (width 0.2) (layer "B.Cu") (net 1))
 (segment (start 46.99 53.11) (end 45.839 54.261) (width 0.2) (layer "B.Cu") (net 1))
 (segment (start 78.994 86.741) (end 85.494 86.741) (width 0.2) (layer "B.Cu") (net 1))
 (segment (start 46.99 60.73) (end 48.26 62) (width 0.2) (layer "B.Cu") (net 1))
 (segment (start 48.379 49.181) (end 48.379 51.721) (width 0.2) (layer "B.Cu") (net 1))
 (segment (start 48.26 67.08) (end 49.53 68.35) (width 0.2) (layer "B.Cu") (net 1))
 (segment (start 50.47 86.13) (end 55.88 91.54) (width 0.2) (layer "B.Cu") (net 1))
 (segment (start 49.53 48.03) (end 48.379 49.181) (width 0.2) (layer "B.Cu") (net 1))
 (segment (start 48.26 62) (end 48.26 67.08) (width 0.2) (layer "B.Cu") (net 1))
 (segment (start 45.839 77.359) (end 46.99 78.51) (width 0.2) (layer "B.Cu") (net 1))
 (segment (start 48.379 46.879) (end 49.53 48.03) (width 0.2) (layer "B.Cu") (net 1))
 (segment (start 46.99 78.51) (end 48.379 79.899) (width 0.2) (layer "B.Cu") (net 1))
 (segment (start 48.379 79.899) (end 48.379 84.979) (width 0.2) (layer "B.Cu") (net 1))
 (segment (start 59.294 85.586) (end 59.294 35.446) (width 0.2) (layer "F.Cu") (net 6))
 (segment (start 59.294 35.446) (end 61.2 33.54) (width 0.2) (layer "F.Cu") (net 6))
 (segment (start 55.88 89) (end 59.294 85.586) (width 0.2) (layer "F.Cu") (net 6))
 (segment (start 57.241 29.679) (end 76.719 29.679) (width 0.2) (layer "F.Cu") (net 3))
 (segment (start 76.719 29.679) (end 80.58 33.54) (width 0.2) (layer "F.Cu") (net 3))
 (segment (start 56 30.92) (end 57.241 29.679) (width 0.2) (layer "F.Cu") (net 3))
 (segment (start 85.494 91.241) (end 86.795 89.94) (width 0.2) (layer "F.Cu") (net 2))
 (segment (start 86.795 62.615) (end 80.58 56.4) (width 0.2) (layer "F.Cu") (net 2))
 (segment (start 78.994 91.241) (end 85.494 91.241) (width 0.2) (layer "F.Cu") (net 2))
 (segment (start 86.795 89.94) (end 86.795 62.615) (width 0.2) (layer "F.Cu") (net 2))
 (segment (start 50.00676 54.261) (end 49.05324 54.261) (width 0.2) (layer "F.Cu") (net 23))
 (segment (start 80.58 71.64) (end 82.486 73.546) (width 0.2) (layer "F.Cu") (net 23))
 (segment (start 74.557 89.338108) (end 74.557 89.50376) (width 0.2) (layer "F.Cu") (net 23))
 (segment (start 55.43024 90.178) (end 50.681 85.42876) (width 0.2) (layer "F.Cu") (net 23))
 (segment (start 82.486 73.546) (end 82.486 81.409108) (width 0.2) (layer "F.Cu") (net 23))
 (segment (start 82.486 81.409108) (end 74.557 89.338108) (width 0.2) (layer "F.Cu") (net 23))
 (segment (start 48.141 53.34876) (end 48.141 51.721) (width 0.2) (layer "F.Cu") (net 23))
 (segment (start 48.141 51.721) (end 46.99 50.57) (width 0.2) (layer "F.Cu") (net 23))
 (segment (start 74.557 89.50376) (end 73.88276 90.178) (width 0.2) (layer "F.Cu") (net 23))
 (segment (start 50.681 54.93524) (end 50.00676 54.261) (width 0.2) (layer "F.Cu") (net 23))
 (segment (start 49.05324 54.261) (end 48.141 53.34876) (width 0.2) (layer "F.Cu") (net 23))
 (segment (start 50.681 85.42876) (end 50.681 54.93524) (width 0.2) (layer "F.Cu") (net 23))
 (segment (start 73.88276 90.178) (end 55.43024 90.178) (width 0.2) (layer "F.Cu") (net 23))
 (segment (start 55.88 86.46) (end 58.893 83.447) (width 0.2) (layer "F.Cu") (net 5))
 (segment (start 58.893 83.447) (end 58.893 33.307) (width 0.2) (layer "F.Cu") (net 5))
 (segment (start 58.893 33.307) (end 61.2 31) (width 0.2) (layer "F.Cu") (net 5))
 (segment (start 68.326 79.054) (end 68.326 89.027) (width 0.2) (layer "F.Cu") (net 36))
 (segment (start 68.35 79.03) (end 68.326 79.054) (width 0.2) (layer "F.Cu") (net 36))
 (segment (start 73.406 79.054) (end 73.406 89.027) (width 0.2) (layer "F.Cu") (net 37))
 (segment (start 73.43 79.03) (end 73.406 79.054) (width 0.2) (layer "F.Cu") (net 37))
 (segment (start 46.99 40.41) (end 48.141 41.561) (width 0.2) (layer "F.Cu") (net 4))
 (segment (start 46.99 40.41) (end 46.99 37.87) (width 0.2) (layer "F.Cu") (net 4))
 (segment (start 55.519 41.561) (end 56 41.08) (width 0.2) (layer "F.Cu") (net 4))
 (segment (start 48.141 41.561) (end 55.519 41.561) (width 0.2) (layer "F.Cu") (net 4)))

